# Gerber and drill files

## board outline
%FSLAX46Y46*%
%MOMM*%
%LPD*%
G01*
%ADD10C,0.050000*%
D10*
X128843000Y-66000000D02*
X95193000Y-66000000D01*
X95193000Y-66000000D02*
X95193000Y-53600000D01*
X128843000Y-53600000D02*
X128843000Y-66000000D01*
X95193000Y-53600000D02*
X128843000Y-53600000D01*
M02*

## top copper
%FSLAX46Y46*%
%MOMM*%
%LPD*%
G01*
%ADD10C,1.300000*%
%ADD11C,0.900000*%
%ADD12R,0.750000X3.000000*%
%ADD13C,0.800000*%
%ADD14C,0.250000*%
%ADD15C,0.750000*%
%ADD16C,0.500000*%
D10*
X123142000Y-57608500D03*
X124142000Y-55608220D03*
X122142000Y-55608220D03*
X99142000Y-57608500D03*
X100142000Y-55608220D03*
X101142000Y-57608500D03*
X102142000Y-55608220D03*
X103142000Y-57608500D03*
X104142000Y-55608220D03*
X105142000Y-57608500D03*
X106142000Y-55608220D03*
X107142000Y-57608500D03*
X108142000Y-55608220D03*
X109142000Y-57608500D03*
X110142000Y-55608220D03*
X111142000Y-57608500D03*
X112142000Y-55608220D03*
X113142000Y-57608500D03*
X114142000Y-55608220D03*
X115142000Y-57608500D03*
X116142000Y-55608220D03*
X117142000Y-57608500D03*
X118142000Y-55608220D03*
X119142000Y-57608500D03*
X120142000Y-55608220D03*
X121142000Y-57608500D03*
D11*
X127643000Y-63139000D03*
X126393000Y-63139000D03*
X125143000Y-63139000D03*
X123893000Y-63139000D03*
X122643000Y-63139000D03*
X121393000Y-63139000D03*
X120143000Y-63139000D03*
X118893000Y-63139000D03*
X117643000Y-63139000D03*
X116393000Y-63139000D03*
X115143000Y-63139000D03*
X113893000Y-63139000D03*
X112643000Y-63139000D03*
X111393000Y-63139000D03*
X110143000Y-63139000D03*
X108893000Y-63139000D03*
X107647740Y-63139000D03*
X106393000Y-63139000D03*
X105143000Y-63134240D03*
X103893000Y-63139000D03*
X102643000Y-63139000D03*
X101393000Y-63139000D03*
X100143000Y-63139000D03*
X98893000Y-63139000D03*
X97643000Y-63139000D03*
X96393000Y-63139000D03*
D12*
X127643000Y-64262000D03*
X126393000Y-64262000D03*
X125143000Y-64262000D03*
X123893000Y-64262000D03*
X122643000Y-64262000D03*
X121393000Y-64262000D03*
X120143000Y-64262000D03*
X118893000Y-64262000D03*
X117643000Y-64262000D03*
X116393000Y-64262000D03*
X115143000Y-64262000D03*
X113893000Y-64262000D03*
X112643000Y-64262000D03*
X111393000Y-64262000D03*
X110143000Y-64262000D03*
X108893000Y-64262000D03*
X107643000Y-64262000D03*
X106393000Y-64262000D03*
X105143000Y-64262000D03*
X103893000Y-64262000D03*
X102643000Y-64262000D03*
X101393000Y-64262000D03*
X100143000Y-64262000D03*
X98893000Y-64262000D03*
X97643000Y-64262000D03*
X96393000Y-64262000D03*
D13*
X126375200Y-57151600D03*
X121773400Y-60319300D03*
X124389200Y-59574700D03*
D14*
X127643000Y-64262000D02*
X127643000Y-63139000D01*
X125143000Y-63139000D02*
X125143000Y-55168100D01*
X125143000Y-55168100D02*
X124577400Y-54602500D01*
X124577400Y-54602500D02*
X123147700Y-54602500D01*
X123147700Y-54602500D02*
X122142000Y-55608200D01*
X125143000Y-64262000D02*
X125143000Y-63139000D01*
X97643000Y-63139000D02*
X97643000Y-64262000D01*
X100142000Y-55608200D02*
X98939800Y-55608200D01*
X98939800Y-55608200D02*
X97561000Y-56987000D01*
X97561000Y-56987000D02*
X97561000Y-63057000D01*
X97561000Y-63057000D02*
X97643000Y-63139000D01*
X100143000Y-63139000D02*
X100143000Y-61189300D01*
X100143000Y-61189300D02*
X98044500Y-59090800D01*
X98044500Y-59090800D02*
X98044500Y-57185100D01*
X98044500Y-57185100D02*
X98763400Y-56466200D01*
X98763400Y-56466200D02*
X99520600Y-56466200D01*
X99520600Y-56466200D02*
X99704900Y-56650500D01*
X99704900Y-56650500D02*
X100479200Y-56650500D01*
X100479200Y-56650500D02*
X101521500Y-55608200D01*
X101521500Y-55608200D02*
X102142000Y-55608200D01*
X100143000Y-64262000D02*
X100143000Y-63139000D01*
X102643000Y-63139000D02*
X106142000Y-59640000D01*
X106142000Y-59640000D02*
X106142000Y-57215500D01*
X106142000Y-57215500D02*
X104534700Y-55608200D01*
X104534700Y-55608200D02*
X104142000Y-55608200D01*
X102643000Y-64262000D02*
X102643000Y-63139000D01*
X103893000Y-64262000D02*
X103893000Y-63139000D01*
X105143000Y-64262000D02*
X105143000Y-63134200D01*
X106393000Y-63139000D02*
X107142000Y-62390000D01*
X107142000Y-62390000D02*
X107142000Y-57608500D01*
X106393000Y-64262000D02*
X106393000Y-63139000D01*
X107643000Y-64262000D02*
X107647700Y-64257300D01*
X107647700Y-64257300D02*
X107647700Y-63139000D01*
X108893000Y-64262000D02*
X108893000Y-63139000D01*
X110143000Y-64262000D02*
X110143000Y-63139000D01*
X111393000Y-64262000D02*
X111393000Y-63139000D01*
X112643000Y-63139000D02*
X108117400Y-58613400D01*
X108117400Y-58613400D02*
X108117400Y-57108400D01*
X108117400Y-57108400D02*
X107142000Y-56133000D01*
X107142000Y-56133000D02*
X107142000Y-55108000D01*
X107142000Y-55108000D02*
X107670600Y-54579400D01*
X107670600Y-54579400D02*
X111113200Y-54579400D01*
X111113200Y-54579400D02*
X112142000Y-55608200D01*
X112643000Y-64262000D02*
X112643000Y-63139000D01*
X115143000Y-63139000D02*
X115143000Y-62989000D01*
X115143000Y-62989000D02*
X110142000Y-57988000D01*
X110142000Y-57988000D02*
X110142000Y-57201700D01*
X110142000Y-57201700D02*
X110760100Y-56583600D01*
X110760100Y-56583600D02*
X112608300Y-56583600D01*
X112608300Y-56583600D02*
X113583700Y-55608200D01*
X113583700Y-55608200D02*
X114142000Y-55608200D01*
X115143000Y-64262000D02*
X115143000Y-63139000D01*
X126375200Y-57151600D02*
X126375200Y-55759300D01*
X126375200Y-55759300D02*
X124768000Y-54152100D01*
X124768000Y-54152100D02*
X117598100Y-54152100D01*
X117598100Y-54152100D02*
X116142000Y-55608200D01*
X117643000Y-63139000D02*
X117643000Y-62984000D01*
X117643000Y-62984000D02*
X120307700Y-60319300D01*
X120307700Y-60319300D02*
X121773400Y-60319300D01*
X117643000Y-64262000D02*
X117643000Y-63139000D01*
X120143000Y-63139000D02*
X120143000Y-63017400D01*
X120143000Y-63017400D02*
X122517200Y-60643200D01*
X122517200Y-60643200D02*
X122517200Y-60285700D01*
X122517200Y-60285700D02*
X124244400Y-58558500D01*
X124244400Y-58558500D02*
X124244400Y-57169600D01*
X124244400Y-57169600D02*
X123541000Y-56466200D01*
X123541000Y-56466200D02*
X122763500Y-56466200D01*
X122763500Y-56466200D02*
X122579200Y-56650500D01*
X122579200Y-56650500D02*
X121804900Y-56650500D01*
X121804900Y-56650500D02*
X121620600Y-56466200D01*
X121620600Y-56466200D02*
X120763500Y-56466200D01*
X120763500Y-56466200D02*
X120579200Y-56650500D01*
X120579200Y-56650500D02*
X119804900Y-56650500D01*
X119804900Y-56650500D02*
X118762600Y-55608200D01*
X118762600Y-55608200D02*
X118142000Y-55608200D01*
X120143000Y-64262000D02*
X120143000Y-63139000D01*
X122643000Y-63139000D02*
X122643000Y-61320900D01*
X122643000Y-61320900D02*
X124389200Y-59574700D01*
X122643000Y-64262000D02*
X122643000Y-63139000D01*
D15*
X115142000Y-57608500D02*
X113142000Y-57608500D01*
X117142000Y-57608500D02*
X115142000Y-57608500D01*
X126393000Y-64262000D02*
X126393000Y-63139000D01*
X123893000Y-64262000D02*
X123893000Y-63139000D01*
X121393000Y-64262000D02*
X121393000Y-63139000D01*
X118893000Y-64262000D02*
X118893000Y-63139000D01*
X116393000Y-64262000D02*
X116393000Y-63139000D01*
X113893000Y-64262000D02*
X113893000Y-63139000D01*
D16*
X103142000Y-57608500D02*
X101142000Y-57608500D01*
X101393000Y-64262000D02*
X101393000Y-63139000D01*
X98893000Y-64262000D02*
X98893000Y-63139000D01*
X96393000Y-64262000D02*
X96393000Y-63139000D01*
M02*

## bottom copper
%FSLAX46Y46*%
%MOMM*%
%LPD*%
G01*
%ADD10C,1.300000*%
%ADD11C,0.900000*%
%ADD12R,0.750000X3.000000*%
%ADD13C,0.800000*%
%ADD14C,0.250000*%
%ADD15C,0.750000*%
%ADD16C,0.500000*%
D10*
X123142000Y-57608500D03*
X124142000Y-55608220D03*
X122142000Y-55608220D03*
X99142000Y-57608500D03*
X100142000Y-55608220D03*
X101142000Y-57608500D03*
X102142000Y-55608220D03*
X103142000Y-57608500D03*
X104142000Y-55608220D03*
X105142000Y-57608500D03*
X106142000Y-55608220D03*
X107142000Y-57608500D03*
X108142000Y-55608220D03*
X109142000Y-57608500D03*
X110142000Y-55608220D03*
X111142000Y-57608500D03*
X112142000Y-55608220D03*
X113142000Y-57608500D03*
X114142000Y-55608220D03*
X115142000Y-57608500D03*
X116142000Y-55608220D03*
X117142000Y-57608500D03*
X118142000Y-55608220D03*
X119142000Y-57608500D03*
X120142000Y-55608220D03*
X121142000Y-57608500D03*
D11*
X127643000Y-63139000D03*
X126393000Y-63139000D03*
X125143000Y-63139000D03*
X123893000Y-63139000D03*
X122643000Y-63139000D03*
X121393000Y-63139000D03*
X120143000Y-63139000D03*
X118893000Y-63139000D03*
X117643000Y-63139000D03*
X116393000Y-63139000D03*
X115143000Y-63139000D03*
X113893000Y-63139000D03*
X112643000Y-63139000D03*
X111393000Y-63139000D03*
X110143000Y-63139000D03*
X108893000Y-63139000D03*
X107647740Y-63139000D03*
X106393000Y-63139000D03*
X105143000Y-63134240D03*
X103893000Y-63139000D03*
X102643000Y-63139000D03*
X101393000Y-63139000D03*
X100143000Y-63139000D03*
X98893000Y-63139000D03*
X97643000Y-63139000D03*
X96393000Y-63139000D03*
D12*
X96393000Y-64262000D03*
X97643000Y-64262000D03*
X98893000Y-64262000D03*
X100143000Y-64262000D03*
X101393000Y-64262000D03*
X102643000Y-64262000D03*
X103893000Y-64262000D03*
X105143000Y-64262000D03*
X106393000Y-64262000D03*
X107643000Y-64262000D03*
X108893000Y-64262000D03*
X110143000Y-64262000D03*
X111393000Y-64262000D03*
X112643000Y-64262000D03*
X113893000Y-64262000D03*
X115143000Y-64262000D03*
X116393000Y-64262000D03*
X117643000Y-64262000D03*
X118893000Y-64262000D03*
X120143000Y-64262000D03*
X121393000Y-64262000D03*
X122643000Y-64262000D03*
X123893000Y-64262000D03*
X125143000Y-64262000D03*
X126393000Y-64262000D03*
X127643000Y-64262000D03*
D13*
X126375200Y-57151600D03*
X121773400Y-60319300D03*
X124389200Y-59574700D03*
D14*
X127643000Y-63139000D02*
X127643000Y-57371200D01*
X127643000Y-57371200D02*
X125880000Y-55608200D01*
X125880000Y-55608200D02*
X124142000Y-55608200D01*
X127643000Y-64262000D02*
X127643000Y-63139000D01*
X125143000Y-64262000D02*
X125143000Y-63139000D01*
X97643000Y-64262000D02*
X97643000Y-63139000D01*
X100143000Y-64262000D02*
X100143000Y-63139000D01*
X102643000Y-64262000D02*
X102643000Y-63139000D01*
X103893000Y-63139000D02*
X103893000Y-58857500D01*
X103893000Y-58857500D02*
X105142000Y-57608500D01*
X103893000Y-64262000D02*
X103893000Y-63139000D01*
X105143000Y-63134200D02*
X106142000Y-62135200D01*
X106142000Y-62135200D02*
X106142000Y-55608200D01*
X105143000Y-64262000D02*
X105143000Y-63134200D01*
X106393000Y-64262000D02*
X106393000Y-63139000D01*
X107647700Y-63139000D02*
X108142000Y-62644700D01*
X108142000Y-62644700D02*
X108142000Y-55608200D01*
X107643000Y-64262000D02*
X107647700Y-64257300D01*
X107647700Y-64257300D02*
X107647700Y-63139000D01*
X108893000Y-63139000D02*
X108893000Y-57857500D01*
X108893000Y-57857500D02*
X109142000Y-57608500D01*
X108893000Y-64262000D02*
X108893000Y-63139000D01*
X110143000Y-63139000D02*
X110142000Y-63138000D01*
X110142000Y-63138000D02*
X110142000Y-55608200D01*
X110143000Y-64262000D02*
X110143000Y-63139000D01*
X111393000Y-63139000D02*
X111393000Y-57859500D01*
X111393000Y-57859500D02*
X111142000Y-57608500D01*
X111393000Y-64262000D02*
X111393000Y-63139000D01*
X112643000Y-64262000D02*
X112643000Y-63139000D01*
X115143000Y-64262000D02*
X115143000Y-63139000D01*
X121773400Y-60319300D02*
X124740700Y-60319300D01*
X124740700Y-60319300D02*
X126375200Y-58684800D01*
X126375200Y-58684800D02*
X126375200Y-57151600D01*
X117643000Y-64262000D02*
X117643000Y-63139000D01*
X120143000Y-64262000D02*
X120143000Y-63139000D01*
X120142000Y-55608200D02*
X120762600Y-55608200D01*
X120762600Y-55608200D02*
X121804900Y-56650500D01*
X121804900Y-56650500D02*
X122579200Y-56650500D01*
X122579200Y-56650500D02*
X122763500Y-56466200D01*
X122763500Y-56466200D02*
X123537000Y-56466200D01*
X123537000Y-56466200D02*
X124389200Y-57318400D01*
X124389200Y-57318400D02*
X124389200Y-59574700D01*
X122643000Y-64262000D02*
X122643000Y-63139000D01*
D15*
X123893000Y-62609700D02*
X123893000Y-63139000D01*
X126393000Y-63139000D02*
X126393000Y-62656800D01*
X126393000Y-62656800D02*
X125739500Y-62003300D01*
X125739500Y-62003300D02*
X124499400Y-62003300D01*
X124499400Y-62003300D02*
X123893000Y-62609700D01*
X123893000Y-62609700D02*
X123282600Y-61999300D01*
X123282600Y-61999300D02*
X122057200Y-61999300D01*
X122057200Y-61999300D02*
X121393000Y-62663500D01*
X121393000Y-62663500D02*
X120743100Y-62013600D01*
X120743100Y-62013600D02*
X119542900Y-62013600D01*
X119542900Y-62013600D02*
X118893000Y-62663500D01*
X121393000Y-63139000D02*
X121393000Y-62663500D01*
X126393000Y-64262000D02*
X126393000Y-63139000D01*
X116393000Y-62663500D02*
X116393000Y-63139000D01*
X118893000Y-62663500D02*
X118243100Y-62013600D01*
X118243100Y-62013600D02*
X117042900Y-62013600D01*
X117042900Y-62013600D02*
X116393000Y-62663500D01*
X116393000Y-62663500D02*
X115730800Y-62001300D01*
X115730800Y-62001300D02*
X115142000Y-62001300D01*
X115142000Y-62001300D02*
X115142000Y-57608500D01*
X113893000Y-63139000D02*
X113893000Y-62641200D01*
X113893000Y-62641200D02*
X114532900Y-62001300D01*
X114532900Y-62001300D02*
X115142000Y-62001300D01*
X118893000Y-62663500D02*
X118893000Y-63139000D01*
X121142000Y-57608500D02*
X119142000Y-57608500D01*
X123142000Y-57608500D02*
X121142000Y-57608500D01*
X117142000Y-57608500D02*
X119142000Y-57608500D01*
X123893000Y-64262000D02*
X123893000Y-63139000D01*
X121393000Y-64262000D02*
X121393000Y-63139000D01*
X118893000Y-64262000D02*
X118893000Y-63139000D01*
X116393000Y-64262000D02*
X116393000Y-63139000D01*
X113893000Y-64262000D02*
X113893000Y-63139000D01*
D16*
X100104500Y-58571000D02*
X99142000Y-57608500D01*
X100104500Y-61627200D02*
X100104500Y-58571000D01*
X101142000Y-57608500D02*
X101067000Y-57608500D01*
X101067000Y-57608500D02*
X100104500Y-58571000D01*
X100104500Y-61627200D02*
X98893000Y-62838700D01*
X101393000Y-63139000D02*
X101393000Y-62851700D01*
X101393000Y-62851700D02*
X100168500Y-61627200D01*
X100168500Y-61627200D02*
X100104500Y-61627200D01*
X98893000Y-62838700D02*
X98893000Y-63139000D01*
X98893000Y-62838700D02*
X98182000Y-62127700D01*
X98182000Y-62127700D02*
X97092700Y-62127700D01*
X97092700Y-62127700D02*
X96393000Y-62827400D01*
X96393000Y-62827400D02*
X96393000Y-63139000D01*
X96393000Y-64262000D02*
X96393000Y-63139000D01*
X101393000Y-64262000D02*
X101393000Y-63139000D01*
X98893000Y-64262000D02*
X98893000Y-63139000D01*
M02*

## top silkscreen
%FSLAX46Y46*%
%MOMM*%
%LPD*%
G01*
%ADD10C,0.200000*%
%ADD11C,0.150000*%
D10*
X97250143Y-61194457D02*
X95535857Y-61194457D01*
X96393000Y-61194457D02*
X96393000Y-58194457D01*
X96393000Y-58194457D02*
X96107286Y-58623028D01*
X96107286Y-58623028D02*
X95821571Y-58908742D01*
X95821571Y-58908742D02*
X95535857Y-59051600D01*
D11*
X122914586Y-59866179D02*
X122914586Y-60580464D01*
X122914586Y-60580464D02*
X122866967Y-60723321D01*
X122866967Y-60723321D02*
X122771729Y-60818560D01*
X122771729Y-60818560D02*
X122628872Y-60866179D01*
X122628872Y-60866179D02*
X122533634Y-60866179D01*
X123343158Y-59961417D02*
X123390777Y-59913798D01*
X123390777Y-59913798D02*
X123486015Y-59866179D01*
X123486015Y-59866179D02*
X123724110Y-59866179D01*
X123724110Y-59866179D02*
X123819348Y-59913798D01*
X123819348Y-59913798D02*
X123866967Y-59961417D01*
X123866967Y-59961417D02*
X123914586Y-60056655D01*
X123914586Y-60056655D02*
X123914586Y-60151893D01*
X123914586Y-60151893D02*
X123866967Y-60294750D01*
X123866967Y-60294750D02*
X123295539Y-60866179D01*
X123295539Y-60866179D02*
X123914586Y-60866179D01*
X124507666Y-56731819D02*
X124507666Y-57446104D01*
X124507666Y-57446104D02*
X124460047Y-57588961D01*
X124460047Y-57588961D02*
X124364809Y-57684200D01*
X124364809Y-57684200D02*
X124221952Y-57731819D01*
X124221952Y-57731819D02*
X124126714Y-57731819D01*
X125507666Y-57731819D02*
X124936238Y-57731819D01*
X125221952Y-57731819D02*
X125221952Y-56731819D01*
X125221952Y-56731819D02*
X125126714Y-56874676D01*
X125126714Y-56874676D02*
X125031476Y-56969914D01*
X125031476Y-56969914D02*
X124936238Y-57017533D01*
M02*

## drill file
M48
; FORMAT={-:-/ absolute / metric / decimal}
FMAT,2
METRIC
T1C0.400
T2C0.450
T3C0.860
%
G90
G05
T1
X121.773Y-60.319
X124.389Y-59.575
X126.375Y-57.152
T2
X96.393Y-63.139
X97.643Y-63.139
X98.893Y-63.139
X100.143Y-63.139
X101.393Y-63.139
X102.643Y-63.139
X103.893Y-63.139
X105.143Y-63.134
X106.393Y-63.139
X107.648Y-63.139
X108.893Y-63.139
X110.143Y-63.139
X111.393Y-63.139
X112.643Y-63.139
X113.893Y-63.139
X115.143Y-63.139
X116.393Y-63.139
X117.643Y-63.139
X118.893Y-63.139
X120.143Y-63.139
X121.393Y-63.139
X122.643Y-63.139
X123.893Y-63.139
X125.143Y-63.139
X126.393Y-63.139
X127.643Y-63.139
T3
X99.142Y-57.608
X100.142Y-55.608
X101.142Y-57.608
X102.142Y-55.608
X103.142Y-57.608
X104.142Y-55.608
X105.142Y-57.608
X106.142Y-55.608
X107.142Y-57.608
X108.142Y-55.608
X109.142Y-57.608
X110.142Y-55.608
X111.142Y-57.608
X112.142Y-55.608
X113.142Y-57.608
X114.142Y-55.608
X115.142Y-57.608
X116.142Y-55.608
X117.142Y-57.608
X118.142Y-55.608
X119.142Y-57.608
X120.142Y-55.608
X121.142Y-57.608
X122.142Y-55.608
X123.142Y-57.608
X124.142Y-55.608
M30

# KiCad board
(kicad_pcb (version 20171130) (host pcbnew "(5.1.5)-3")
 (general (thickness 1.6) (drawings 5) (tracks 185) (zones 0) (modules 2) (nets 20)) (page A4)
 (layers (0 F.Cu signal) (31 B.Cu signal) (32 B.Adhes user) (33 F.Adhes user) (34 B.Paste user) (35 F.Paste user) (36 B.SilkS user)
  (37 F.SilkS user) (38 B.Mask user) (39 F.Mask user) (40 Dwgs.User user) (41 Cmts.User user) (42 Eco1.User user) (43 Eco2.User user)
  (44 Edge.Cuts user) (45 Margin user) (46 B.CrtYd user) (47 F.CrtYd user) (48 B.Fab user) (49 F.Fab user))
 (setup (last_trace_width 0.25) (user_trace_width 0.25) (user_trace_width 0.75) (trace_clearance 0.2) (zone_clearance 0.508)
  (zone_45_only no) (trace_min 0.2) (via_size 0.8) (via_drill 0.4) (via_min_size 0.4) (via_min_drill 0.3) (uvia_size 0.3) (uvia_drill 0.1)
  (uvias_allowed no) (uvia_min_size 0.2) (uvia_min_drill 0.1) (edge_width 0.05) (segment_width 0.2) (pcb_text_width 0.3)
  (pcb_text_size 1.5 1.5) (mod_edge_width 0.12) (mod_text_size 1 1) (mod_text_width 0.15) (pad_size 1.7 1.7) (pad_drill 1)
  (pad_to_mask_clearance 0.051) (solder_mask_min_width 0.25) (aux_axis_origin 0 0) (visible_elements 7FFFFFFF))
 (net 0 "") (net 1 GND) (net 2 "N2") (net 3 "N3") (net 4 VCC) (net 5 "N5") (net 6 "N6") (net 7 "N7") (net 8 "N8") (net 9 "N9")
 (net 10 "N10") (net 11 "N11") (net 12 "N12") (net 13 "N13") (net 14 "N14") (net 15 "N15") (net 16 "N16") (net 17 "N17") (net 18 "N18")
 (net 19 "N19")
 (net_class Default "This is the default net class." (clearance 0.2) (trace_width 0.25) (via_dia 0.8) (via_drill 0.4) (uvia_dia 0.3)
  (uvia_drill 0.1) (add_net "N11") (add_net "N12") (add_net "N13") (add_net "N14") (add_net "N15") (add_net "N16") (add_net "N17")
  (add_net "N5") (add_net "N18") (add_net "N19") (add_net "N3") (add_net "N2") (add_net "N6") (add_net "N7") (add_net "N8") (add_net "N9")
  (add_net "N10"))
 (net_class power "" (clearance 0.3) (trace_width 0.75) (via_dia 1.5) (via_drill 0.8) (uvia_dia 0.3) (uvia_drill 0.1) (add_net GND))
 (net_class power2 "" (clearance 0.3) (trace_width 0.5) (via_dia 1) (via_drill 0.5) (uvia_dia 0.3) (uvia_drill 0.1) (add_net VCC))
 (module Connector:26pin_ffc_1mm (layer F.Cu) (at 124.142 52.8955 180)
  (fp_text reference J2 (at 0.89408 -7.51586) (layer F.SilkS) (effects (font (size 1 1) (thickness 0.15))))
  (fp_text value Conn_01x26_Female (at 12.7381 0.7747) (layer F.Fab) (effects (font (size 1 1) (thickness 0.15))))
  (pad 25 thru_hole circle (at 1 -4.713 180) (size 1.3 1.3) (drill 0.86) (layers *.Cu *.Mask) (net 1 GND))
  (pad 26 thru_hole circle (at 0 -2.71272 180) (size 1.3 1.3) (drill 0.86) (layers *.Cu *.Mask) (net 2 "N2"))
  (pad 24 thru_hole circle (at 2 -2.71272 180) (size 1.3 1.3) (drill 0.86) (layers *.Cu *.Mask) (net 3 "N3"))
  (pad 1 thru_hole circle (at 25 -4.713 180) (size 1.3 1.3) (drill 0.86) (layers *.Cu *.Mask) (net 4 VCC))
  (pad 2 thru_hole circle (at 24 -2.71272 180) (size 1.3 1.3) (drill 0.86) (layers *.Cu *.Mask) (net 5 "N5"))
  (pad 3 thru_hole circle (at 23 -4.713 180) (size 1.3 1.3) (drill 0.86) (layers *.Cu *.Mask) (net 4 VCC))
  (pad 4 thru_hole circle (at 22 -2.71272 180) (size 1.3 1.3) (drill 0.86) (layers *.Cu *.Mask) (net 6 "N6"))
  (pad 5 thru_hole circle (at 21 -4.713 180) (size 1.3 1.3) (drill 0.86) (layers *.Cu *.Mask) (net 4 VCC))
  (pad 6 thru_hole circle (at 20 -2.71272 180) (size 1.3 1.3) (drill 0.86) (layers *.Cu *.Mask) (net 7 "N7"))
  (pad 7 thru_hole circle (at 19 -4.713 180) (size 1.3 1.3) (drill 0.86) (layers *.Cu *.Mask) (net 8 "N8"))
  (pad 8 thru_hole circle (at 18 -2.71272 180) (size 1.3 1.3) (drill 0.86) (layers *.Cu *.Mask) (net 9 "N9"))
  (pad 9 thru_hole circle (at 17 -4.713 180) (size 1.3 1.3) (drill 0.86) (layers *.Cu *.Mask) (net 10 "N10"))
  (pad 10 thru_hole circle (at 16 -2.71272 180) (size 1.3 1.3) (drill 0.86) (layers *.Cu *.Mask) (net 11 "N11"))
  (pad 11 thru_hole circle (at 15 -4.713 180) (size 1.3 1.3) (drill 0.86) (layers *.Cu *.Mask) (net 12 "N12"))
  (pad 12 thru_hole circle (at 14 -2.71272 180) (size 1.3 1.3) (drill 0.86) (layers *.Cu *.Mask) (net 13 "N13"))
  (pad 13 thru_hole circle (at 13 -4.713 180) (size 1.3 1.3) (drill 0.86) (layers *.Cu *.Mask) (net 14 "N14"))
  (pad 14 thru_hole circle (at 12 -2.71272 180) (size 1.3 1.3) (drill 0.86) (layers *.Cu *.Mask) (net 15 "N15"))
  (pad 15 thru_hole circle (at 11 -4.713 180) (size 1.3 1.3) (drill 0.86) (layers *.Cu *.Mask) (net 1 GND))
  (pad 16 thru_hole circle (at 10 -2.71272 180) (size 1.3 1.3) (drill 0.86) (layers *.Cu *.Mask) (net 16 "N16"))
  (pad 17 thru_hole circle (at 9 -4.713 180) (size 1.3 1.3) (drill 0.86) (layers *.Cu *.Mask) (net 1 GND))
  (pad 18 thru_hole circle (at 8 -2.71272 180) (size 1.3 1.3) (drill 0.86) (layers *.Cu *.Mask) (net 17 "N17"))
  (pad 19 thru_hole circle (at 7 -4.713 180) (size 1.3 1.3) (drill 0.86) (layers *.Cu *.Mask) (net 1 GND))
  (pad 20 thru_hole circle (at 6 -2.71272 180) (size 1.3 1.3) (drill 0.86) (layers *.Cu *.Mask) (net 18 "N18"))
  (pad 21 thru_hole circle (at 5 -4.713 180) (size 1.3 1.3) (drill 0.86) (layers *.Cu *.Mask) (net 1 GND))
  (pad 22 thru_hole circle (at 4 -2.71272 180) (size 1.3 1.3) (drill 0.86) (layers *.Cu *.Mask) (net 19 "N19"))
  (pad 23 thru_hole circle (at 3 -4.713 180) (size 1.3 1.3) (drill 0.86) (layers *.Cu *.Mask) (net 1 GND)))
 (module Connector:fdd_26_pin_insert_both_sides (layer F.Cu) (at 96.393 64.389)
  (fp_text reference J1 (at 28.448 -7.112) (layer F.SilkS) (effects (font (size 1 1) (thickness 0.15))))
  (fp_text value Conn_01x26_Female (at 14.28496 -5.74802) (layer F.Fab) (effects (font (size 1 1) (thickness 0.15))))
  (pad 26 thru_hole circle (at 31.25 -1.25) (size 0.9 0.9) (drill 0.45) (layers *.Cu *.Mask) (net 2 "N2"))
  (pad 25 thru_hole circle (at 30 -1.25) (size 0.9 0.9) (drill 0.45) (layers *.Cu *.Mask) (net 1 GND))
  (pad 24 thru_hole circle (at 28.75 -1.25) (size 0.9 0.9) (drill 0.45) (layers *.Cu *.Mask) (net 3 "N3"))
  (pad 23 thru_hole circle (at 27.5 -1.25) (size 0.9 0.9) (drill 0.45) (layers *.Cu *.Mask) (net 1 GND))
  (pad 22 thru_hole circle (at 26.25 -1.25) (size 0.9 0.9) (drill 0.45) (layers *.Cu *.Mask) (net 19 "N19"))
  (pad 21 thru_hole circle (at 25 -1.25) (size 0.9 0.9) (drill 0.45) (layers *.Cu *.Mask) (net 1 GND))
  (pad 20 thru_hole circle (at 23.75 -1.25) (size 0.9 0.9) (drill 0.45) (layers *.Cu *.Mask) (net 18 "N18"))
  (pad 19 thru_hole circle (at 22.5 -1.25) (size 0.9 0.9) (drill 0.45) (layers *.Cu *.Mask) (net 1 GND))
  (pad 18 thru_hole circle (at 21.25 -1.25) (size 0.9 0.9) (drill 0.45) (layers *.Cu *.Mask) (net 17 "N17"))
  (pad 17 thru_hole circle (at 20 -1.25) (size 0.9 0.9) (drill 0.45) (layers *.Cu *.Mask) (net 1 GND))
  (pad 16 thru_hole circle (at 18.75 -1.25) (size 0.9 0.9) (drill 0.45) (layers *.Cu *.Mask) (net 16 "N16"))
  (pad 15 thru_hole circle (at 17.5 -1.25 90) (size 0.9 0.9) (drill 0.45) (layers *.Cu *.Mask) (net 1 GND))
  (pad 14 thru_hole circle (at 16.25 -1.25) (size 0.9 0.9) (drill 0.45) (layers *.Cu *.Mask) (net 15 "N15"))
  (pad 13 thru_hole circle (at 15 -1.25) (size 0.9 0.9) (drill 0.45) (layers *.Cu *.Mask) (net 14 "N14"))
  (pad 12 thru_hole circle (at 13.75 -1.25) (size 0.9 0.9) (drill 0.45) (layers *.Cu *.Mask) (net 13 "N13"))
  (pad 11 thru_hole circle (at 12.5 -1.25) (size 0.9 0.9) (drill 0.45) (layers *.Cu *.Mask) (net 12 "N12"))
  (pad 10 thru_hole circle (at 11.25474 -1.25) (size 0.9 0.9) (drill 0.45) (layers *.Cu *.Mask) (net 11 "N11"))
  (pad 9 thru_hole circle (at 10 -1.25) (size 0.9 0.9) (drill 0.45) (layers *.Cu *.Mask) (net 10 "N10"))
  (pad 8 thru_hole circle (at 8.75 -1.25476) (size 0.9 0.9) (drill 0.45) (layers *.Cu *.Mask) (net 9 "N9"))
  (pad 7 thru_hole circle (at 7.5 -1.25) (size 0.9 0.9) (drill 0.45) (layers *.Cu *.Mask) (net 8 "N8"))
  (pad 6 thru_hole circle (at 6.25 -1.25) (size 0.9 0.9) (drill 0.45) (layers *.Cu *.Mask) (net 7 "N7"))
  (pad 5 thru_hole circle (at 5 -1.25) (size 0.9 0.9) (drill 0.45) (layers *.Cu *.Mask) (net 4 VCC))
  (pad 4 thru_hole circle (at 3.75 -1.25) (size 0.9 0.9) (drill 0.45) (layers *.Cu *.Mask) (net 6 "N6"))
  (pad 3 thru_hole circle (at 2.5 -1.25) (size 0.9 0.9) (drill 0.45) (layers *.Cu *.Mask) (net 4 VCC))
  (pad 2 thru_hole circle (at 1.25 -1.25 90) (size 0.9 0.9) (drill 0.45) (layers *.Cu *.Mask) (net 5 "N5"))
  (pad 1 thru_hole circle (at 0 -1.25) (size 0.9 0.9) (drill 0.45) (layers *.Cu *.Mask) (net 4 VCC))
  (pad 26 connect rect (at 31.25 -0.127) (size 0.75 3) (layers F.Cu F.Mask) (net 2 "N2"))
  (pad 25 connect rect (at 30 -0.127) (size 0.75 3) (layers F.Cu F.Mask) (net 1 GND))
  (pad 24 connect rect (at 28.75 -0.127) (size 0.75 3) (layers F.Cu F.Mask) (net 3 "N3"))
  (pad 23 connect rect (at 27.5 -0.127) (size 0.75 3) (layers F.Cu F.Mask) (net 1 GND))
  (pad 22 connect rect (at 26.25 -0.127) (size 0.75 3) (layers F.Cu F.Mask) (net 19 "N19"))
  (pad 21 connect rect (at 25 -0.127) (size 0.75 3) (layers F.Cu F.Mask) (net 1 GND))
  (pad 20 connect rect (at 23.75 -0.127) (size 0.75 3) (layers F.Cu F.Mask) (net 18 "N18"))
  (pad 19 connect rect (at 22.5 -0.127) (size 0.75 3) (layers F.Cu F.Mask) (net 1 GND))
  (pad 18 connect rect (at 21.25 -0.127) (size 0.75 3) (layers F.Cu F.Mask) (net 17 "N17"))
  (pad 17 connect rect (at 20 -0.127) (size 0.75 3) (layers F.Cu F.Mask) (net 1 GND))
  (pad 16 connect rect (at 18.75 -0.127) (size 0.75 3) (layers F.Cu F.Mask) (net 16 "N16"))
  (pad 15 connect rect (at 17.5 -0.127) (size 0.75 3) (layers F.Cu F.Mask) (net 1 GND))
  (pad 14 connect rect (at 16.25 -0.127) (size 0.75 3) (layers F.Cu F.Mask) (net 15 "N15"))
  (pad 13 connect rect (at 15 -0.127) (size 0.75 3) (layers F.Cu F.Mask) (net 14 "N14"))
  (pad 12 connect rect (at 13.75 -0.127) (size 0.75 3) (layers F.Cu F.Mask) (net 13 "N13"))
  (pad 11 connect rect (at 12.5 -0.127) (size 0.75 3) (layers F.Cu F.Mask) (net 12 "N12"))
  (pad 10 connect rect (at 11.25 -0.127) (size 0.75 3) (layers F.Cu F.Mask) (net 11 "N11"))
  (pad 9 connect rect (at 10 -0.127) (size 0.75 3) (layers F.Cu F.Mask) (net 10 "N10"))
  (pad 8 connect rect (at 8.75 -0.127) (size 0.75 3) (layers F.Cu F.Mask) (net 9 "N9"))
  (pad 7 connect rect (at 7.5 -0.127) (size 0.75 3) (layers F.Cu F.Mask) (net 8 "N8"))
  (pad 6 connect rect (at 6.25 -0.127) (size 0.75 3) (layers F.Cu F.Mask) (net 7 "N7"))
  (pad 5 connect rect (at 5 -0.127) (size 0.75 3) (layers F.Cu F.Mask) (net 4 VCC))
  (pad 4 connect rect (at 3.75 -0.127) (size 0.75 3) (layers F.Cu F.Mask) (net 6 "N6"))
  (pad 3 connect rect (at 2.5 -0.127) (size 0.75 3) (layers F.Cu F.Mask) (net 4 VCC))
  (pad 2 connect rect (at 1.25 -0.127) (size 0.75 3) (layers F.Cu F.Mask) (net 5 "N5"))
  (pad 1 connect rect (at 0 -0.127) (size 0.75 3) (layers F.Cu F.Mask) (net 4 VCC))
  (pad 1 connect rect (at 0 -0.127) (size 0.75 3) (layers B.Cu B.Mask) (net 4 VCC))
  (pad 2 connect rect (at 1.25 -0.127) (size 0.75 3) (layers B.Cu B.Mask) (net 5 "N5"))
  (pad 3 connect rect (at 2.5 -0.127) (size 0.75 3) (layers B.Cu B.Mask) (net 4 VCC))
  (pad 4 connect rect (at 3.75 -0.127) (size 0.75 3) (layers B.Cu B.Mask) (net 6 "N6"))
  (pad 5 connect rect (at 5 -0.127) (size 0.75 3) (layers B.Cu B.Mask) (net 4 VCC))
  (pad 6 connect rect (at 6.25 -0.127) (size 0.75 3) (layers B.Cu B.Mask) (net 7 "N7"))
  (pad 7 connect rect (at 7.5 -0.127) (size 0.75 3) (layers B.Cu B.Mask) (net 8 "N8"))
  (pad 8 connect rect (at 8.75 -0.127) (size 0.75 3) (layers B.Cu B.Mask) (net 9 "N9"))
  (pad 9 connect rect (at 10 -0.127) (size 0.75 3) (layers B.Cu B.Mask) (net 10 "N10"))
  (pad 10 connect rect (at 11.25 -0.127) (size 0.75 3) (layers B.Cu B.Mask) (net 11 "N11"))
  (pad 11 connect rect (at 12.5 -0.127) (size 0.75 3) (layers B.Cu B.Mask) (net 12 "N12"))
  (pad 12 connect rect (at 13.75 -0.127) (size 0.75 3) (layers B.Cu B.Mask) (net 13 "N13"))
  (pad 13 connect rect (at 15 -0.127) (size 0.75 3) (layers B.Cu B.Mask) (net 14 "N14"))
  (pad 14 connect rect (at 16.25 -0.127) (size 0.75 3) (layers B.Cu B.Mask) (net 15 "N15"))
  (pad 15 connect rect (at 17.5 -0.127) (size 0.75 3) (layers B.Cu B.Mask) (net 1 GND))
  (pad 16 connect rect (at 18.75 -0.127) (size 0.75 3) (layers B.Cu B.Mask) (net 16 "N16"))
  (pad 17 connect rect (at 20 -0.127) (size 0.75 3) (layers B.Cu B.Mask) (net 1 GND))
  (pad 18 connect rect (at 21.25 -0.127) (size 0.75 3) (layers B.Cu B.Mask) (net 17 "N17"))
  (pad 19 connect rect (at 22.5 -0.127) (size 0.75 3) (layers B.Cu B.Mask) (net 1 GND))
  (pad 20 connect rect (at 23.75 -0.127) (size 0.75 3) (layers B.Cu B.Mask) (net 18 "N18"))
  (pad 21 connect rect (at 25 -0.127) (size 0.75 3) (layers B.Cu B.Mask) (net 1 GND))
  (pad 22 connect rect (at 26.25 -0.127) (size 0.75 3) (layers B.Cu B.Mask) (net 19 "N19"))
  (pad 23 connect rect (at 27.5 -0.127) (size 0.75 3) (layers B.Cu B.Mask) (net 1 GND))
  (pad 24 connect rect (at 28.75 -0.127) (size 0.75 3) (layers B.Cu B.Mask) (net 3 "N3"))
  (pad 25 connect rect (at 30 -0.127) (size 0.75 3) (layers B.Cu B.Mask) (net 1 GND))
  (pad 26 connect rect (at 31.25 -0.127) (size 0.75 3) (layers B.Cu B.Mask) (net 2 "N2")))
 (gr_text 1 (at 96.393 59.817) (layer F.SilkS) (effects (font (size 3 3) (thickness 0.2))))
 (gr_line (start 128.843 66) (end 95.193 66) (layer Edge.Cuts) (width 0.05))
 (gr_line (start 95.193 66) (end 95.193 53.6) (layer Edge.Cuts) (width 0.05))
 (gr_line (start 128.843 53.6) (end 128.843 66) (layer Edge.Cuts) (width 0.05))
 (gr_line (start 95.193 53.6) (end 128.843 53.6) (layer Edge.Cuts) (width 0.05))
 (segment (start 127.643 63.139) (end 127.643 57.3712) (width 0.25) (layer B.Cu) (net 2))
 (segment (start 127.643 57.3712) (end 125.88 55.6082) (width 0.25) (layer B.Cu) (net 2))
 (segment (start 125.88 55.6082) (end 124.142 55.6082) (width 0.25) (layer B.Cu) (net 2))
 (segment (start 127.643 64.262) (end 127.643 63.139) (width 0.25) (layer B.Cu) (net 2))
 (segment (start 127.643 64.262) (end 127.643 63.139) (width 0.25) (layer F.Cu) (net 2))
 (segment (start 125.143 63.139) (end 125.143 55.1681) (width 0.25) (layer F.Cu) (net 3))
 (segment (start 125.143 55.1681) (end 124.5774 54.6025) (width 0.25) (layer F.Cu) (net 3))
 (segment (start 124.5774 54.6025) (end 123.1477 54.6025) (width 0.25) (layer F.Cu) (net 3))
 (segment (start 123.1477 54.6025) (end 122.142 55.6082) (width 0.25) (layer F.Cu) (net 3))
 (segment (start 125.143 64.262) (end 125.143 63.139) (width 0.25) (layer F.Cu) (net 3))
 (segment (start 125.143 64.262) (end 125.143 63.139) (width 0.25) (layer B.Cu) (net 3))
 (segment (start 97.643 63.139) (end 97.643 64.262) (width 0.25) (layer F.Cu) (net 5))
 (segment (start 100.142 55.6082) (end 98.9398 55.6082) (width 0.25) (layer F.Cu) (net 5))
 (segment (start 98.9398 55.6082) (end 97.561 56.987) (width 0.25) (layer F.Cu) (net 5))
 (segment (start 97.561 56.987) (end 97.561 63.057) (width 0.25) (layer F.Cu) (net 5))
 (segment (start 97.561 63.057) (end 97.643 63.139) (width 0.25) (layer F.Cu) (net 5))
 (segment (start 97.643 64.262) (end 97.643 63.139) (width 0.25) (layer B.Cu) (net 5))
 (segment (start 100.143 64.262) (end 100.143 63.139) (width 0.25) (layer B.Cu) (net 6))
 (segment (start 100.143 63.139) (end 100.143 61.1893) (width 0.25) (layer F.Cu) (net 6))
 (segment (start 100.143 61.1893) (end 98.0445 59.0908) (width 0.25) (layer F.Cu) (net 6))
 (segment (start 98.0445 59.0908) (end 98.0445 57.1851) (width 0.25) (layer F.Cu) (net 6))
 (segment (start 98.0445 57.1851) (end 98.7634 56.4662) (width 0.25) (layer F.Cu) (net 6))
 (segment (start 98.7634 56.4662) (end 99.5206 56.4662) (width 0.25) (layer F.Cu) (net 6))
 (segment (start 99.5206 56.4662) (end 99.7049 56.6505) (width 0.25) (layer F.Cu) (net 6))
 (segment (start 99.7049 56.6505) (end 100.4792 56.6505) (width 0.25) (layer F.Cu) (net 6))
 (segment (start 100.4792 56.6505) (end 101.5215 55.6082) (width 0.25) (layer F.Cu) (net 6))
 (segment (start 101.5215 55.6082) (end 102.142 55.6082) (width 0.25) (layer F.Cu) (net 6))
 (segment (start 100.143 64.262) (end 100.143 63.139) (width 0.25) (layer F.Cu) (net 6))
 (segment (start 102.643 63.139) (end 106.142 59.64) (width 0.25) (layer F.Cu) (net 7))
 (segment (start 106.142 59.64) (end 106.142 57.2155) (width 0.25) (layer F.Cu) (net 7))
 (segment (start 106.142 57.2155) (end 104.5347 55.6082) (width 0.25) (layer F.Cu) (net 7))
 (segment (start 104.5347 55.6082) (end 104.142 55.6082) (width 0.25) (layer F.Cu) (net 7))
 (segment (start 102.643 64.262) (end 102.643 63.139) (width 0.25) (layer F.Cu) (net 7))
 (segment (start 102.643 64.262) (end 102.643 63.139) (width 0.25) (layer B.Cu) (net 7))
 (segment (start 103.893 63.139) (end 103.893 58.8575) (width 0.25) (layer B.Cu) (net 8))
 (segment (start 103.893 58.8575) (end 105.142 57.6085) (width 0.25) (layer B.Cu) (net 8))
 (segment (start 103.893 64.262) (end 103.893 63.139) (width 0.25) (layer B.Cu) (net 8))
 (segment (start 103.893 64.262) (end 103.893 63.139) (width 0.25) (layer F.Cu) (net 8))
 (segment (start 105.143 63.1342) (end 106.142 62.1352) (width 0.25) (layer B.Cu) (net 9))
 (segment (start 106.142 62.1352) (end 106.142 55.6082) (width 0.25) (layer B.Cu) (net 9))
 (segment (start 105.143 64.262) (end 105.143 63.1342) (width 0.25) (layer B.Cu) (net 9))
 (segment (start 105.143 64.262) (end 105.143 63.1342) (width 0.25) (layer F.Cu) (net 9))
 (segment (start 106.393 63.139) (end 107.142 62.39) (width 0.25) (layer F.Cu) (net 10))
 (segment (start 107.142 62.39) (end 107.142 57.6085) (width 0.25) (layer F.Cu) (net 10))
 (segment (start 106.393 64.262) (end 106.393 63.139) (width 0.25) (layer F.Cu) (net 10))
 (segment (start 106.393 64.262) (end 106.393 63.139) (width 0.25) (layer B.Cu) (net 10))
 (segment (start 107.6477 63.139) (end 108.142 62.6447) (width 0.25) (layer B.Cu) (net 11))
 (segment (start 108.142 62.6447) (end 108.142 55.6082) (width 0.25) (layer B.Cu) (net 11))
 (segment (start 107.643 64.262) (end 107.6477 64.2573) (width 0.25) (layer B.Cu) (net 11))
 (segment (start 107.6477 64.2573) (end 107.6477 63.139) (width 0.25) (layer B.Cu) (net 11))
 (segment (start 107.643 64.262) (end 107.6477 64.2573) (width 0.25) (layer F.Cu) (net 11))
 (segment (start 107.6477 64.2573) (end 107.6477 63.139) (width 0.25) (layer F.Cu) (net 11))
 (segment (start 108.893 63.139) (end 108.893 57.8575) (width 0.25) (layer B.Cu) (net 12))
 (segment (start 108.893 57.8575) (end 109.142 57.6085) (width 0.25) (layer B.Cu) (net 12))
 (segment (start 108.893 64.262) (end 108.893 63.139) (width 0.25) (layer B.Cu) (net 12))
 (segment (start 108.893 64.262) (end 108.893 63.139) (width 0.25) (layer F.Cu) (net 12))
 (segment (start 110.143 63.139) (end 110.142 63.138) (width 0.25) (layer B.Cu) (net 13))
 (segment (start 110.142 63.138) (end 110.142 55.6082) (width 0.25) (layer B.Cu) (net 13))
 (segment (start 110.143 64.262) (end 110.143 63.139) (width 0.25) (layer B.Cu) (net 13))
 (segment (start 110.143 64.262) (end 110.143 63.139) (width 0.25) (layer F.Cu) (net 13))
 (segment (start 111.393 63.139) (end 111.393 57.8595) (width 0.25) (layer B.Cu) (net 14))
 (segment (start 111.393 57.8595) (end 111.142 57.6085) (width 0.25) (layer B.Cu) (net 14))
 (segment (start 111.393 64.262) (end 111.393 63.139) (width 0.25) (layer B.Cu) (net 14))
 (segment (start 111.393 64.262) (end 111.393 63.139) (width 0.25) (layer F.Cu) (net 14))
 (segment (start 112.643 63.139) (end 108.1174 58.6134) (width 0.25) (layer F.Cu) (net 15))
 (segment (start 108.1174 58.6134) (end 108.1174 57.1084) (width 0.25) (layer F.Cu) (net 15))
 (segment (start 108.1174 57.1084) (end 107.142 56.133) (width 0.25) (layer F.Cu) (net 15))
 (segment (start 107.142 56.133) (end 107.142 55.108) (width 0.25) (layer F.Cu) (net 15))
 (segment (start 107.142 55.108) (end 107.6706 54.5794) (width 0.25) (layer F.Cu) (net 15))
 (segment (start 107.6706 54.5794) (end 111.1132 54.5794) (width 0.25) (layer F.Cu) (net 15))
 (segment (start 111.1132 54.5794) (end 112.142 55.6082) (width 0.25) (layer F.Cu) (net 15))
 (segment (start 112.643 64.262) (end 112.643 63.139) (width 0.25) (layer F.Cu) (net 15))
 (segment (start 112.643 64.262) (end 112.643 63.139) (width 0.25) (layer B.Cu) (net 15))
 (segment (start 115.143 63.139) (end 115.143 62.989) (width 0.25) (layer F.Cu) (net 16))
 (segment (start 115.143 62.989) (end 110.142 57.988) (width 0.25) (layer F.Cu) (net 16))
 (segment (start 110.142 57.988) (end 110.142 57.2017) (width 0.25) (layer F.Cu) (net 16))
 (segment (start 110.142 57.2017) (end 110.7601 56.5836) (width 0.25) (layer F.Cu) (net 16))
 (segment (start 110.7601 56.5836) (end 112.6083 56.5836) (width 0.25) (layer F.Cu) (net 16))
 (segment (start 112.6083 56.5836) (end 113.5837 55.6082) (width 0.25) (layer F.Cu) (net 16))
 (segment (start 113.5837 55.6082) (end 114.142 55.6082) (width 0.25) (layer F.Cu) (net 16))
 (segment (start 115.143 64.262) (end 115.143 63.139) (width 0.25) (layer F.Cu) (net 16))
 (segment (start 115.143 64.262) (end 115.143 63.139) (width 0.25) (layer B.Cu) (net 16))
 (segment (start 126.3752 57.1516) (end 126.3752 55.7593) (width 0.25) (layer F.Cu) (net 17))
 (segment (start 126.3752 55.7593) (end 124.768 54.1521) (width 0.25) (layer F.Cu) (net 17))
 (segment (start 124.768 54.1521) (end 117.5981 54.1521) (width 0.25) (layer F.Cu) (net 17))
 (segment (start 117.5981 54.1521) (end 116.142 55.6082) (width 0.25) (layer F.Cu) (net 17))
 (segment (start 121.7734 60.3193) (end 124.7407 60.3193) (width 0.25) (layer B.Cu) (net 17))
 (segment (start 124.7407 60.3193) (end 126.3752 58.6848) (width 0.25) (layer B.Cu) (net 17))
 (segment (start 126.3752 58.6848) (end 126.3752 57.1516) (width 0.25) (layer B.Cu) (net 17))
 (segment (start 117.643 63.139) (end 117.643 62.984) (width 0.25) (layer F.Cu) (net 17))
 (segment (start 117.643 62.984) (end 120.3077 60.3193) (width 0.25) (layer F.Cu) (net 17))
 (segment (start 120.3077 60.3193) (end 121.7734 60.3193) (width 0.25) (layer F.Cu) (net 17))
 (segment (start 117.643 64.262) (end 117.643 63.139) (width 0.25) (layer F.Cu) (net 17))
 (segment (start 117.643 64.262) (end 117.643 63.139) (width 0.25) (layer B.Cu) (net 17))
 (via (at 126.3752 57.1516) (size 0.8) (layers F.Cu B.Cu) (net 17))
 (via (at 121.7734 60.3193) (size 0.8) (layers F.Cu B.Cu) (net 17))
 (segment (start 120.143 63.139) (end 120.143 63.0174) (width 0.25) (layer F.Cu) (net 18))
 (segment (start 120.143 63.0174) (end 122.5172 60.6432) (width 0.25) (layer F.Cu) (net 18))
 (segment (start 122.5172 60.6432) (end 122.5172 60.2857) (width 0.25) (layer F.Cu) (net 18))
 (segment (start 122.5172 60.2857) (end 124.2444 58.5585) (width 0.25) (layer F.Cu) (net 18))
 (segment (start 124.2444 58.5585) (end 124.2444 57.1696) (width 0.25) (layer F.Cu) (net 18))
 (segment (start 124.2444 57.1696) (end 123.541 56.4662) (width 0.25) (layer F.Cu) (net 18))
 (segment (start 123.541 56.4662) (end 122.7635 56.4662) (width 0.25) (layer F.Cu) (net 18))
 (segment (start 122.7635 56.4662) (end 122.5792 56.6505) (width 0.25) (layer F.Cu) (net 18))
 (segment (start 122.5792 56.6505) (end 121.8049 56.6505) (width 0.25) (layer F.Cu) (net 18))
 (segment (start 121.8049 56.6505) (end 121.6206 56.4662) (width 0.25) (layer F.Cu) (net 18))
 (segment (start 121.6206 56.4662) (end 120.7635 56.4662) (width 0.25) (layer F.Cu) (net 18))
 (segment (start 120.7635 56.4662) (end 120.5792 56.6505) (width 0.25) (layer F.Cu) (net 18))
 (segment (start 120.5792 56.6505) (end 119.8049 56.6505) (width 0.25) (layer F.Cu) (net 18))
 (segment (start 119.8049 56.6505) (end 118.7626 55.6082) (width 0.25) (layer F.Cu) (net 18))
 (segment (start 118.7626 55.6082) (end 118.142 55.6082) (width 0.25) (layer F.Cu) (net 18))
 (segment (start 120.143 64.262) (end 120.143 63.139) (width 0.25) (layer F.Cu) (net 18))
 (segment (start 120.143 64.262) (end 120.143 63.139) (width 0.25) (layer B.Cu) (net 18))
 (segment (start 122.643 63.139) (end 122.643 61.3209) (width 0.25) (layer F.Cu) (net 19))
 (segment (start 122.643 61.3209) (end 124.3892 59.5747) (width 0.25) (layer F.Cu) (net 19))
 (segment (start 120.142 55.6082) (end 120.7626 55.6082) (width 0.25) (layer B.Cu) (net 19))
 (segment (start 120.7626 55.6082) (end 121.8049 56.6505) (width 0.25) (layer B.Cu) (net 19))
 (segment (start 121.8049 56.6505) (end 122.5792 56.6505) (width 0.25) (layer B.Cu) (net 19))
 (segment (start 122.5792 56.6505) (end 122.7635 56.4662) (width 0.25) (layer B.Cu) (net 19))
 (segment (start 122.7635 56.4662) (end 123.537 56.4662) (width 0.25) (layer B.Cu) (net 19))
 (segment (start 123.537 56.4662) (end 124.3892 57.3184) (width 0.25) (layer B.Cu) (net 19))
 (segment (start 124.3892 57.3184) (end 124.3892 59.5747) (width 0.25) (layer B.Cu) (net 19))
 (segment (start 122.643 64.262) (end 122.643 63.139) (width 0.25) (layer F.Cu) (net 19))
 (segment (start 122.643 64.262) (end 122.643 63.139) (width 0.25) (layer B.Cu) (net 19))
 (via (at 124.3892 59.5747) (size 0.8) (layers F.Cu B.Cu) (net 19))
 (segment (start 123.893 62.6097) (end 123.893 63.139) (width 0.75) (layer B.Cu) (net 1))
 (segment (start 126.393 63.139) (end 126.393 62.6568) (width 0.75) (layer B.Cu) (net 1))
 (segment (start 126.393 62.6568) (end 125.7395 62.0033) (width 0.75) (layer B.Cu) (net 1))
 (segment (start 125.7395 62.0033) (end 124.4994 62.0033) (width 0.75) (layer B.Cu) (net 1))
 (segment (start 124.4994 62.0033) (end 123.893 62.6097) (width 0.75) (layer B.Cu) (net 1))
 (segment (start 123.893 62.6097) (end 123.2826 61.9993) (width 0.75) (layer B.Cu) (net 1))
 (segment (start 123.2826 61.9993) (end 122.0572 61.9993) (width 0.75) (layer B.Cu) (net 1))
 (segment (start 122.0572 61.9993) (end 121.393 62.6635) (width 0.75) (layer B.Cu) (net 1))
 (segment (start 121.393 62.6635) (end 120.7431 62.0136) (width 0.75) (layer B.Cu) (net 1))
 (segment (start 120.7431 62.0136) (end 119.5429 62.0136) (width 0.75) (layer B.Cu) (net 1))
 (segment (start 119.5429 62.0136) (end 118.893 62.6635) (width 0.75) (layer B.Cu) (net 1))
 (segment (start 121.393 63.139) (end 121.393 62.6635) (width 0.75) (layer B.Cu) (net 1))
 (segment (start 126.393 64.262) (end 126.393 63.139) (width 0.75) (layer B.Cu) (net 1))
 (segment (start 116.393 62.6635) (end 116.393 63.139) (width 0.75) (layer B.Cu) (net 1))
 (segment (start 118.893 62.6635) (end 118.2431 62.0136) (width 0.75) (layer B.Cu) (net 1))
 (segment (start 118.2431 62.0136) (end 117.0429 62.0136) (width 0.75) (layer B.Cu) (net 1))
 (segment (start 117.0429 62.0136) (end 116.393 62.6635) (width 0.75) (layer B.Cu) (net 1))
 (segment (start 116.393 62.6635) (end 115.7308 62.0013) (width 0.75) (layer B.Cu) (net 1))
 (segment (start 115.7308 62.0013) (end 115.142 62.0013) (width 0.75) (layer B.Cu) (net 1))
 (segment (start 115.142 62.0013) (end 115.142 57.6085) (width 0.75) (layer B.Cu) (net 1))
 (segment (start 113.893 63.139) (end 113.893 62.6412) (width 0.75) (layer B.Cu) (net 1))
 (segment (start 113.893 62.6412) (end 114.5329 62.0013) (width 0.75) (layer B.Cu) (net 1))
 (segment (start 114.5329 62.0013) (end 115.142 62.0013) (width 0.75) (layer B.Cu) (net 1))
 (segment (start 118.893 62.6635) (end 118.893 63.139) (width 0.75) (layer B.Cu) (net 1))
 (segment (start 115.142 57.6085) (end 113.142 57.6085) (width 0.75) (layer F.Cu) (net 1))
 (segment (start 117.142 57.6085) (end 115.142 57.6085) (width 0.75) (layer F.Cu) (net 1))
 (segment (start 121.142 57.6085) (end 119.142 57.6085) (width 0.75) (layer B.Cu) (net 1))
 (segment (start 123.142 57.6085) (end 121.142 57.6085) (width 0.75) (layer B.Cu) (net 1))
 (segment (start 117.142 57.6085) (end 119.142 57.6085) (width 0.75) (layer B.Cu) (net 1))
 (segment (start 123.893 64.262) (end 123.893 63.139) (width 0.75) (layer B.Cu) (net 1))
 (segment (start 121.393 64.262) (end 121.393 63.139) (width 0.75) (layer B.Cu) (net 1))
 (segment (start 118.893 64.262) (end 118.893 63.139) (width 0.75) (layer B.Cu) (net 1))
 (segment (start 116.393 64.262) (end 116.393 63.139) (width 0.75) (layer B.Cu) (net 1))
 (segment (start 113.893 64.262) (end 113.893 63.139) (width 0.75) (layer B.Cu) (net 1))
 (segment (start 126.393 64.262) (end 126.393 63.139) (width 0.75) (layer F.Cu) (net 1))
 (segment (start 123.893 64.262) (end 123.893 63.139) (width 0.75) (layer F.Cu) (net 1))
 (segment (start 121.393 64.262) (end 121.393 63.139) (width 0.75) (layer F.Cu) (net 1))
 (segment (start 118.893 64.262) (end 118.893 63.139) (width 0.75) (layer F.Cu) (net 1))
 (segment (start 116.393 64.262) (end 116.393 63.139) (width 0.75) (layer F.Cu) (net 1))
 (segment (start 113.893 64.262) (end 113.893 63.139) (width 0.75) (layer F.Cu) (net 1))
 (segment (start 100.1045 58.571) (end 99.142 57.6085) (width 0.5) (layer B.Cu) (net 4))
 (segment (start 100.1045 61.6272) (end 100.1045 58.571) (width 0.5) (layer B.Cu) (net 4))
 (segment (start 101.142 57.6085) (end 101.067 57.6085) (width 0.5) (layer B.Cu) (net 4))
 (segment (start 101.067 57.6085) (end 100.1045 58.571) (width 0.5) (layer B.Cu) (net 4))
 (segment (start 100.1045 61.6272) (end 98.893 62.8387) (width 0.5) (layer B.Cu) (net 4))
 (segment (start 101.393 63.139) (end 101.393 62.8517) (width 0.5) (layer B.Cu) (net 4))
 (segment (start 101.393 62.8517) (end 100.1685 61.6272) (width 0.5) (layer B.Cu) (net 4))
 (segment (start 100.1685 61.6272) (end 100.1045 61.6272) (width 0.5) (layer B.Cu) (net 4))
 (segment (start 98.893 62.8387) (end 98.893 63.139) (width 0.5) (layer B.Cu) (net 4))
 (segment (start 98.893 62.8387) (end 98.182 62.1277) (width 0.5) (layer B.Cu) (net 4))
 (segment (start 98.182 62.1277) (end 97.0927 62.1277) (width 0.5) (layer B.Cu) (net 4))
 (segment (start 97.0927 62.1277) (end 96.393 62.8274) (width 0.5) (layer B.Cu) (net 4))
 (segment (start 96.393 62.8274) (end 96.393 63.139) (width 0.5) (layer B.Cu) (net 4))
 (segment (start 96.393 64.262) (end 96.393 63.139) (width 0.5) (layer B.Cu) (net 4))
 (segment (start 101.393 64.262) (end 101.393 63.139) (width 0.5) (layer B.Cu) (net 4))
 (segment (start 103.142 57.6085) (end 101.142 57.6085) (width 0.5) (layer F.Cu) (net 4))
 (segment (start 98.893 64.262) (end 98.893 63.139) (width 0.5) (layer B.Cu) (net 4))
 (segment (start 101.393 64.262) (end 101.393 63.139) (width 0.5) (layer F.Cu) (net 4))
 (segment (start 98.893 64.262) (end 98.893 63.139) (width 0.5) (layer F.Cu) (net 4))
 (segment (start 96.393 64.262) (end 96.393 63.139) (width 0.5) (layer F.Cu) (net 4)))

